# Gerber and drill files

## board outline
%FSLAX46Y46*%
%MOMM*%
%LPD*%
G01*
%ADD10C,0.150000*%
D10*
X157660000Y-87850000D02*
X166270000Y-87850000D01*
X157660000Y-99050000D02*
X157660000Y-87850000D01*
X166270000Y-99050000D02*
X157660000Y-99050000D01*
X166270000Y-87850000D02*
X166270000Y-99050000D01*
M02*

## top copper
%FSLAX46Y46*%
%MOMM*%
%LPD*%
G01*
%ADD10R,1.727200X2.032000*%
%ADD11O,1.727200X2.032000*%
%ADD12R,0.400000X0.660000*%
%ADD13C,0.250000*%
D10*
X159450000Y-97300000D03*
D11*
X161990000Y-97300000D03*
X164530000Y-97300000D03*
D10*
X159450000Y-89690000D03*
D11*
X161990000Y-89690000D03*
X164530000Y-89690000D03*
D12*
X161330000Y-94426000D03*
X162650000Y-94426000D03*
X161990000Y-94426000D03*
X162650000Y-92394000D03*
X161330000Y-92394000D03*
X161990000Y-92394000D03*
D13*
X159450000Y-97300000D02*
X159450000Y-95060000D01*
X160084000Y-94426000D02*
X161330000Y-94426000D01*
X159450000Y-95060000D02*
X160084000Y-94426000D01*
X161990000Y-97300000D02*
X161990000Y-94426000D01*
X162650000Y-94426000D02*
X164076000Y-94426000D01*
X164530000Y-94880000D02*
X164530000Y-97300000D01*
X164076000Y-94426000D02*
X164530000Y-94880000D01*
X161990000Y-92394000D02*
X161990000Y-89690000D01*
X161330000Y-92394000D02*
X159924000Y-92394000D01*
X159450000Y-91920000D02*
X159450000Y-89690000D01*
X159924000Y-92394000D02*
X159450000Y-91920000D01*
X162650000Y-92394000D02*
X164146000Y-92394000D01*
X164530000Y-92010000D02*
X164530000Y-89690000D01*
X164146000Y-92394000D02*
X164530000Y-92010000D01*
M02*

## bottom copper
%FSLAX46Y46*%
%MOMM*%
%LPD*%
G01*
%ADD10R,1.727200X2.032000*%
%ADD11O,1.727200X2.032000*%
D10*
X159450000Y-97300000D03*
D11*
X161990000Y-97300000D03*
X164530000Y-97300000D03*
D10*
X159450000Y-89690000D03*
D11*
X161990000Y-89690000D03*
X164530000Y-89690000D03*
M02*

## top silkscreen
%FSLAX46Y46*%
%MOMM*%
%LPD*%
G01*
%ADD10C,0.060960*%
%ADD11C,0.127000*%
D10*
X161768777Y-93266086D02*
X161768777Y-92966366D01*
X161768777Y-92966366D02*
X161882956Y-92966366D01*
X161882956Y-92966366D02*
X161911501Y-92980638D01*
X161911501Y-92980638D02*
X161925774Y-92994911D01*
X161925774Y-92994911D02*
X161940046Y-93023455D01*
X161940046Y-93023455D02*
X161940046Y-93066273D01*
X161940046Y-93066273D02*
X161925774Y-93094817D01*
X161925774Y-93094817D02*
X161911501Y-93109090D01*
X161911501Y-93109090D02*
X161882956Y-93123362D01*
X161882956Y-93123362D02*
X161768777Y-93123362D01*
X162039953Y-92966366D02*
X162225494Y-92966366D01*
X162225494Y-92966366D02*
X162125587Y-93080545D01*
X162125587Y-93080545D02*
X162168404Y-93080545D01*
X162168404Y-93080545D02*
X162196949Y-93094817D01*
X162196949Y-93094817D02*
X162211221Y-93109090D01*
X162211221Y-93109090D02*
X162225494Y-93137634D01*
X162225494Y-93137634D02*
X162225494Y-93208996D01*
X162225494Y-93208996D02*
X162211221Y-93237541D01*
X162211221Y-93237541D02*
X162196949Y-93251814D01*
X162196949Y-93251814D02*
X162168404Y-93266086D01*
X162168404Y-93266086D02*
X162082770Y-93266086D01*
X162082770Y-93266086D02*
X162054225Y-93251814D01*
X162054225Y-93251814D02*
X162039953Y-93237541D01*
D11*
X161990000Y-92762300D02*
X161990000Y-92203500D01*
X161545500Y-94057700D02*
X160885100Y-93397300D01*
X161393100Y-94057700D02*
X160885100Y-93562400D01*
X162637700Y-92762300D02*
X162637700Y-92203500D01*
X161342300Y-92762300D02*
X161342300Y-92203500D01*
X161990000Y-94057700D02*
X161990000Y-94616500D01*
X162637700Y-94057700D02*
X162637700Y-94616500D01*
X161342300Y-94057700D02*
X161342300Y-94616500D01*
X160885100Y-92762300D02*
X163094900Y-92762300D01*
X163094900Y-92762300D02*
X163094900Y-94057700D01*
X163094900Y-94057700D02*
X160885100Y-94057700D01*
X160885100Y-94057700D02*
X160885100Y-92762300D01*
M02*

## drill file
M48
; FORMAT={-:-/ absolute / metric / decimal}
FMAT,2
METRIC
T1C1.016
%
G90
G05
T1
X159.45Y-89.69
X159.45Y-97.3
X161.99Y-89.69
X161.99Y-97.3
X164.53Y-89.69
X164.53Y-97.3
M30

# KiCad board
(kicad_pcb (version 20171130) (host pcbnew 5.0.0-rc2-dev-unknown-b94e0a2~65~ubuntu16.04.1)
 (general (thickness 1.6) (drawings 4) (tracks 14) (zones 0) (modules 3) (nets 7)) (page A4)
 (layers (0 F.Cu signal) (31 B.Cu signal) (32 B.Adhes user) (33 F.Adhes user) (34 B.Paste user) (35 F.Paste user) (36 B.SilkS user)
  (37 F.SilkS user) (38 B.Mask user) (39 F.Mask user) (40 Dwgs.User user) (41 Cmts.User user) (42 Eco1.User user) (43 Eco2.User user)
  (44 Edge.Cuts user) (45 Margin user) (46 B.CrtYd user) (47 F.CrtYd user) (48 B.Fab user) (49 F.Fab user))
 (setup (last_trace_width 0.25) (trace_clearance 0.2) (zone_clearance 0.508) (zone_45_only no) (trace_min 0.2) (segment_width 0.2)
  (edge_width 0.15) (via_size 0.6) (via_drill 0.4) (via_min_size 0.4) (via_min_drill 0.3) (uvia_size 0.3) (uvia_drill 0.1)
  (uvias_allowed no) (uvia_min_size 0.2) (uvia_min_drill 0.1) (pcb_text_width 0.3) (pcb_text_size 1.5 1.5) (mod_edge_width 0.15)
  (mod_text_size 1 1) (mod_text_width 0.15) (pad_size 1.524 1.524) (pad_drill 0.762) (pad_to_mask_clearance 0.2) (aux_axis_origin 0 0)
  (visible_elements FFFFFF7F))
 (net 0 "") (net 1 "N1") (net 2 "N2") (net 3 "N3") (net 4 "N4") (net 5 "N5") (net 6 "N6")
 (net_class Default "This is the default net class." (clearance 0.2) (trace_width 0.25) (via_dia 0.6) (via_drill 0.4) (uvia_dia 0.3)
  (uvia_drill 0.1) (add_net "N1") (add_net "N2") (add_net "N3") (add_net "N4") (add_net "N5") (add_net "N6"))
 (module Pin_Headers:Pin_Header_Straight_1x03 (layer B.Cu) (at 159.45 97.3 270)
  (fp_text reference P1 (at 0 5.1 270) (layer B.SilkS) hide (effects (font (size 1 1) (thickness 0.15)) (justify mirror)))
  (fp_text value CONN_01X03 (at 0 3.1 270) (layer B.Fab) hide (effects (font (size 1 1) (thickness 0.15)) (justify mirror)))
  (pad 1 thru_hole rect (at 0 0 270) (size 2.032 1.7272) (drill 1.016) (layers *.Cu *.Mask B.SilkS) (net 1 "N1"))
  (pad 2 thru_hole oval (at 0 -2.54 270) (size 2.032 1.7272) (drill 1.016) (layers *.Cu *.Mask B.SilkS) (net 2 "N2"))
  (pad 3 thru_hole oval (at 0 -5.08 270) (size 2.032 1.7272) (drill 1.016) (layers *.Cu *.Mask B.SilkS) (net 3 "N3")))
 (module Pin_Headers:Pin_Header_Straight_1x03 (layer B.Cu) (at 159.45 89.69 270)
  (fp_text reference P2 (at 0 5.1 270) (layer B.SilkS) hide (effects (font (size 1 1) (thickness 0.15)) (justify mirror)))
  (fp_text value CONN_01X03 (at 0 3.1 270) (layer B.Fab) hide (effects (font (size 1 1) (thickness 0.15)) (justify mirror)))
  (pad 1 thru_hole rect (at 0 0 270) (size 2.032 1.7272) (drill 1.016) (layers *.Cu *.Mask B.SilkS) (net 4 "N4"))
  (pad 2 thru_hole oval (at 0 -2.54 270) (size 2.032 1.7272) (drill 1.016) (layers *.Cu *.Mask B.SilkS) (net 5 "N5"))
  (pad 3 thru_hole oval (at 0 -5.08 270) (size 2.032 1.7272) (drill 1.016) (layers *.Cu *.Mask B.SilkS) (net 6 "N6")))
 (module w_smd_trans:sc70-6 (layer F.Cu) (at 161.99 93.41)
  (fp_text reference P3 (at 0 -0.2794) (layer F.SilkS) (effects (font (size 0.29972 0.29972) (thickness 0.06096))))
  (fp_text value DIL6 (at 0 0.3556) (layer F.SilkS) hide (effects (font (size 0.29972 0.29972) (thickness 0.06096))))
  (fp_line (start 0 -0.6477) (end 0 -1.2065) (layer F.SilkS) (width 0.127))
  (fp_line (start -0.4445 0.6477) (end -1.1049 -0.0127) (layer F.SilkS) (width 0.127))
  (fp_line (start -0.5969 0.6477) (end -1.1049 0.1524) (layer F.SilkS) (width 0.127))
  (fp_line (start 0.6477 -0.6477) (end 0.6477 -1.2065) (layer F.SilkS) (width 0.127))
  (fp_line (start -0.6477 -0.6477) (end -0.6477 -1.2065) (layer F.SilkS) (width 0.127))
  (fp_line (start 0 0.6477) (end 0 1.2065) (layer F.SilkS) (width 0.127))
  (fp_line (start 0.6477 0.6477) (end 0.6477 1.2065) (layer F.SilkS) (width 0.127))
  (fp_line (start -0.6477 0.6477) (end -0.6477 1.2065) (layer F.SilkS) (width 0.127))
  (fp_line (start -1.1049 -0.6477) (end 1.1049 -0.6477) (layer F.SilkS) (width 0.127))
  (fp_line (start 1.1049 -0.6477) (end 1.1049 0.6477) (layer F.SilkS) (width 0.127))
  (fp_line (start 1.1049 0.6477) (end -1.1049 0.6477) (layer F.SilkS) (width 0.127))
  (fp_line (start -1.1049 0.6477) (end -1.1049 -0.6477) (layer F.SilkS) (width 0.127))
  (pad 1 smd rect (at -0.66 1.016) (size 0.4 0.66) (layers F.Cu F.Paste F.Mask) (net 1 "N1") (clearance 0.2))
  (pad 3 smd rect (at 0.66 1.016) (size 0.4 0.66) (layers F.Cu F.Paste F.Mask) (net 3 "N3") (clearance 0.2))
  (pad 2 smd rect (at 0 1.016) (size 0.4 0.66) (layers F.Cu F.Paste F.Mask) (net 2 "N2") (clearance 0.2))
  (pad 4 smd rect (at 0.66 -1.016) (size 0.4 0.66) (layers F.Cu F.Paste F.Mask) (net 6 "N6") (clearance 0.2))
  (pad 6 smd rect (at -0.66 -1.016) (size 0.4 0.66) (layers F.Cu F.Paste F.Mask) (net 4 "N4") (clearance 0.2))
  (pad 5 smd rect (at 0 -1.016) (size 0.4 0.66) (layers F.Cu F.Paste F.Mask) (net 5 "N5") (clearance 0.2)))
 (gr_line (start 157.66 87.85) (end 166.27 87.85) (angle 90) (layer Edge.Cuts) (width 0.15))
 (gr_line (start 157.66 99.05) (end 157.66 87.85) (angle 90) (layer Edge.Cuts) (width 0.15))
 (gr_line (start 166.27 99.05) (end 157.66 99.05) (angle 90) (layer Edge.Cuts) (width 0.15))
 (gr_line (start 166.27 87.85) (end 166.27 99.05) (angle 90) (layer Edge.Cuts) (width 0.15))
 (segment (start 159.45 97.3) (end 159.45 95.06) (width 0.25) (layer F.Cu) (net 1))
 (segment (start 160.084 94.426) (end 161.33 94.426) (width 0.25) (layer F.Cu) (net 1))
 (segment (start 159.45 95.06) (end 160.084 94.426) (width 0.25) (layer F.Cu) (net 1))
 (segment (start 161.99 97.3) (end 161.99 94.426) (width 0.25) (layer F.Cu) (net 2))
 (segment (start 162.65 94.426) (end 164.076 94.426) (width 0.25) (layer F.Cu) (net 3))
 (segment (start 164.53 94.88) (end 164.53 97.3) (width 0.25) (layer F.Cu) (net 3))
 (segment (start 164.076 94.426) (end 164.53 94.88) (width 0.25) (layer F.Cu) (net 3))
 (segment (start 161.99 92.394) (end 161.99 89.69) (width 0.25) (layer F.Cu) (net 5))
 (segment (start 161.33 92.394) (end 159.924 92.394) (width 0.25) (layer F.Cu) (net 4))
 (segment (start 159.45 91.92) (end 159.45 89.69) (width 0.25) (layer F.Cu) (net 4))
 (segment (start 159.924 92.394) (end 159.45 91.92) (width 0.25) (layer F.Cu) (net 4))
 (segment (start 162.65 92.394) (end 164.146 92.394) (width 0.25) (layer F.Cu) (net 6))
 (segment (start 164.53 92.01) (end 164.53 89.69) (width 0.25) (layer F.Cu) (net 6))
 (segment (start 164.146 92.394) (end 164.53 92.01) (width 0.25) (layer F.Cu) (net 6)))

